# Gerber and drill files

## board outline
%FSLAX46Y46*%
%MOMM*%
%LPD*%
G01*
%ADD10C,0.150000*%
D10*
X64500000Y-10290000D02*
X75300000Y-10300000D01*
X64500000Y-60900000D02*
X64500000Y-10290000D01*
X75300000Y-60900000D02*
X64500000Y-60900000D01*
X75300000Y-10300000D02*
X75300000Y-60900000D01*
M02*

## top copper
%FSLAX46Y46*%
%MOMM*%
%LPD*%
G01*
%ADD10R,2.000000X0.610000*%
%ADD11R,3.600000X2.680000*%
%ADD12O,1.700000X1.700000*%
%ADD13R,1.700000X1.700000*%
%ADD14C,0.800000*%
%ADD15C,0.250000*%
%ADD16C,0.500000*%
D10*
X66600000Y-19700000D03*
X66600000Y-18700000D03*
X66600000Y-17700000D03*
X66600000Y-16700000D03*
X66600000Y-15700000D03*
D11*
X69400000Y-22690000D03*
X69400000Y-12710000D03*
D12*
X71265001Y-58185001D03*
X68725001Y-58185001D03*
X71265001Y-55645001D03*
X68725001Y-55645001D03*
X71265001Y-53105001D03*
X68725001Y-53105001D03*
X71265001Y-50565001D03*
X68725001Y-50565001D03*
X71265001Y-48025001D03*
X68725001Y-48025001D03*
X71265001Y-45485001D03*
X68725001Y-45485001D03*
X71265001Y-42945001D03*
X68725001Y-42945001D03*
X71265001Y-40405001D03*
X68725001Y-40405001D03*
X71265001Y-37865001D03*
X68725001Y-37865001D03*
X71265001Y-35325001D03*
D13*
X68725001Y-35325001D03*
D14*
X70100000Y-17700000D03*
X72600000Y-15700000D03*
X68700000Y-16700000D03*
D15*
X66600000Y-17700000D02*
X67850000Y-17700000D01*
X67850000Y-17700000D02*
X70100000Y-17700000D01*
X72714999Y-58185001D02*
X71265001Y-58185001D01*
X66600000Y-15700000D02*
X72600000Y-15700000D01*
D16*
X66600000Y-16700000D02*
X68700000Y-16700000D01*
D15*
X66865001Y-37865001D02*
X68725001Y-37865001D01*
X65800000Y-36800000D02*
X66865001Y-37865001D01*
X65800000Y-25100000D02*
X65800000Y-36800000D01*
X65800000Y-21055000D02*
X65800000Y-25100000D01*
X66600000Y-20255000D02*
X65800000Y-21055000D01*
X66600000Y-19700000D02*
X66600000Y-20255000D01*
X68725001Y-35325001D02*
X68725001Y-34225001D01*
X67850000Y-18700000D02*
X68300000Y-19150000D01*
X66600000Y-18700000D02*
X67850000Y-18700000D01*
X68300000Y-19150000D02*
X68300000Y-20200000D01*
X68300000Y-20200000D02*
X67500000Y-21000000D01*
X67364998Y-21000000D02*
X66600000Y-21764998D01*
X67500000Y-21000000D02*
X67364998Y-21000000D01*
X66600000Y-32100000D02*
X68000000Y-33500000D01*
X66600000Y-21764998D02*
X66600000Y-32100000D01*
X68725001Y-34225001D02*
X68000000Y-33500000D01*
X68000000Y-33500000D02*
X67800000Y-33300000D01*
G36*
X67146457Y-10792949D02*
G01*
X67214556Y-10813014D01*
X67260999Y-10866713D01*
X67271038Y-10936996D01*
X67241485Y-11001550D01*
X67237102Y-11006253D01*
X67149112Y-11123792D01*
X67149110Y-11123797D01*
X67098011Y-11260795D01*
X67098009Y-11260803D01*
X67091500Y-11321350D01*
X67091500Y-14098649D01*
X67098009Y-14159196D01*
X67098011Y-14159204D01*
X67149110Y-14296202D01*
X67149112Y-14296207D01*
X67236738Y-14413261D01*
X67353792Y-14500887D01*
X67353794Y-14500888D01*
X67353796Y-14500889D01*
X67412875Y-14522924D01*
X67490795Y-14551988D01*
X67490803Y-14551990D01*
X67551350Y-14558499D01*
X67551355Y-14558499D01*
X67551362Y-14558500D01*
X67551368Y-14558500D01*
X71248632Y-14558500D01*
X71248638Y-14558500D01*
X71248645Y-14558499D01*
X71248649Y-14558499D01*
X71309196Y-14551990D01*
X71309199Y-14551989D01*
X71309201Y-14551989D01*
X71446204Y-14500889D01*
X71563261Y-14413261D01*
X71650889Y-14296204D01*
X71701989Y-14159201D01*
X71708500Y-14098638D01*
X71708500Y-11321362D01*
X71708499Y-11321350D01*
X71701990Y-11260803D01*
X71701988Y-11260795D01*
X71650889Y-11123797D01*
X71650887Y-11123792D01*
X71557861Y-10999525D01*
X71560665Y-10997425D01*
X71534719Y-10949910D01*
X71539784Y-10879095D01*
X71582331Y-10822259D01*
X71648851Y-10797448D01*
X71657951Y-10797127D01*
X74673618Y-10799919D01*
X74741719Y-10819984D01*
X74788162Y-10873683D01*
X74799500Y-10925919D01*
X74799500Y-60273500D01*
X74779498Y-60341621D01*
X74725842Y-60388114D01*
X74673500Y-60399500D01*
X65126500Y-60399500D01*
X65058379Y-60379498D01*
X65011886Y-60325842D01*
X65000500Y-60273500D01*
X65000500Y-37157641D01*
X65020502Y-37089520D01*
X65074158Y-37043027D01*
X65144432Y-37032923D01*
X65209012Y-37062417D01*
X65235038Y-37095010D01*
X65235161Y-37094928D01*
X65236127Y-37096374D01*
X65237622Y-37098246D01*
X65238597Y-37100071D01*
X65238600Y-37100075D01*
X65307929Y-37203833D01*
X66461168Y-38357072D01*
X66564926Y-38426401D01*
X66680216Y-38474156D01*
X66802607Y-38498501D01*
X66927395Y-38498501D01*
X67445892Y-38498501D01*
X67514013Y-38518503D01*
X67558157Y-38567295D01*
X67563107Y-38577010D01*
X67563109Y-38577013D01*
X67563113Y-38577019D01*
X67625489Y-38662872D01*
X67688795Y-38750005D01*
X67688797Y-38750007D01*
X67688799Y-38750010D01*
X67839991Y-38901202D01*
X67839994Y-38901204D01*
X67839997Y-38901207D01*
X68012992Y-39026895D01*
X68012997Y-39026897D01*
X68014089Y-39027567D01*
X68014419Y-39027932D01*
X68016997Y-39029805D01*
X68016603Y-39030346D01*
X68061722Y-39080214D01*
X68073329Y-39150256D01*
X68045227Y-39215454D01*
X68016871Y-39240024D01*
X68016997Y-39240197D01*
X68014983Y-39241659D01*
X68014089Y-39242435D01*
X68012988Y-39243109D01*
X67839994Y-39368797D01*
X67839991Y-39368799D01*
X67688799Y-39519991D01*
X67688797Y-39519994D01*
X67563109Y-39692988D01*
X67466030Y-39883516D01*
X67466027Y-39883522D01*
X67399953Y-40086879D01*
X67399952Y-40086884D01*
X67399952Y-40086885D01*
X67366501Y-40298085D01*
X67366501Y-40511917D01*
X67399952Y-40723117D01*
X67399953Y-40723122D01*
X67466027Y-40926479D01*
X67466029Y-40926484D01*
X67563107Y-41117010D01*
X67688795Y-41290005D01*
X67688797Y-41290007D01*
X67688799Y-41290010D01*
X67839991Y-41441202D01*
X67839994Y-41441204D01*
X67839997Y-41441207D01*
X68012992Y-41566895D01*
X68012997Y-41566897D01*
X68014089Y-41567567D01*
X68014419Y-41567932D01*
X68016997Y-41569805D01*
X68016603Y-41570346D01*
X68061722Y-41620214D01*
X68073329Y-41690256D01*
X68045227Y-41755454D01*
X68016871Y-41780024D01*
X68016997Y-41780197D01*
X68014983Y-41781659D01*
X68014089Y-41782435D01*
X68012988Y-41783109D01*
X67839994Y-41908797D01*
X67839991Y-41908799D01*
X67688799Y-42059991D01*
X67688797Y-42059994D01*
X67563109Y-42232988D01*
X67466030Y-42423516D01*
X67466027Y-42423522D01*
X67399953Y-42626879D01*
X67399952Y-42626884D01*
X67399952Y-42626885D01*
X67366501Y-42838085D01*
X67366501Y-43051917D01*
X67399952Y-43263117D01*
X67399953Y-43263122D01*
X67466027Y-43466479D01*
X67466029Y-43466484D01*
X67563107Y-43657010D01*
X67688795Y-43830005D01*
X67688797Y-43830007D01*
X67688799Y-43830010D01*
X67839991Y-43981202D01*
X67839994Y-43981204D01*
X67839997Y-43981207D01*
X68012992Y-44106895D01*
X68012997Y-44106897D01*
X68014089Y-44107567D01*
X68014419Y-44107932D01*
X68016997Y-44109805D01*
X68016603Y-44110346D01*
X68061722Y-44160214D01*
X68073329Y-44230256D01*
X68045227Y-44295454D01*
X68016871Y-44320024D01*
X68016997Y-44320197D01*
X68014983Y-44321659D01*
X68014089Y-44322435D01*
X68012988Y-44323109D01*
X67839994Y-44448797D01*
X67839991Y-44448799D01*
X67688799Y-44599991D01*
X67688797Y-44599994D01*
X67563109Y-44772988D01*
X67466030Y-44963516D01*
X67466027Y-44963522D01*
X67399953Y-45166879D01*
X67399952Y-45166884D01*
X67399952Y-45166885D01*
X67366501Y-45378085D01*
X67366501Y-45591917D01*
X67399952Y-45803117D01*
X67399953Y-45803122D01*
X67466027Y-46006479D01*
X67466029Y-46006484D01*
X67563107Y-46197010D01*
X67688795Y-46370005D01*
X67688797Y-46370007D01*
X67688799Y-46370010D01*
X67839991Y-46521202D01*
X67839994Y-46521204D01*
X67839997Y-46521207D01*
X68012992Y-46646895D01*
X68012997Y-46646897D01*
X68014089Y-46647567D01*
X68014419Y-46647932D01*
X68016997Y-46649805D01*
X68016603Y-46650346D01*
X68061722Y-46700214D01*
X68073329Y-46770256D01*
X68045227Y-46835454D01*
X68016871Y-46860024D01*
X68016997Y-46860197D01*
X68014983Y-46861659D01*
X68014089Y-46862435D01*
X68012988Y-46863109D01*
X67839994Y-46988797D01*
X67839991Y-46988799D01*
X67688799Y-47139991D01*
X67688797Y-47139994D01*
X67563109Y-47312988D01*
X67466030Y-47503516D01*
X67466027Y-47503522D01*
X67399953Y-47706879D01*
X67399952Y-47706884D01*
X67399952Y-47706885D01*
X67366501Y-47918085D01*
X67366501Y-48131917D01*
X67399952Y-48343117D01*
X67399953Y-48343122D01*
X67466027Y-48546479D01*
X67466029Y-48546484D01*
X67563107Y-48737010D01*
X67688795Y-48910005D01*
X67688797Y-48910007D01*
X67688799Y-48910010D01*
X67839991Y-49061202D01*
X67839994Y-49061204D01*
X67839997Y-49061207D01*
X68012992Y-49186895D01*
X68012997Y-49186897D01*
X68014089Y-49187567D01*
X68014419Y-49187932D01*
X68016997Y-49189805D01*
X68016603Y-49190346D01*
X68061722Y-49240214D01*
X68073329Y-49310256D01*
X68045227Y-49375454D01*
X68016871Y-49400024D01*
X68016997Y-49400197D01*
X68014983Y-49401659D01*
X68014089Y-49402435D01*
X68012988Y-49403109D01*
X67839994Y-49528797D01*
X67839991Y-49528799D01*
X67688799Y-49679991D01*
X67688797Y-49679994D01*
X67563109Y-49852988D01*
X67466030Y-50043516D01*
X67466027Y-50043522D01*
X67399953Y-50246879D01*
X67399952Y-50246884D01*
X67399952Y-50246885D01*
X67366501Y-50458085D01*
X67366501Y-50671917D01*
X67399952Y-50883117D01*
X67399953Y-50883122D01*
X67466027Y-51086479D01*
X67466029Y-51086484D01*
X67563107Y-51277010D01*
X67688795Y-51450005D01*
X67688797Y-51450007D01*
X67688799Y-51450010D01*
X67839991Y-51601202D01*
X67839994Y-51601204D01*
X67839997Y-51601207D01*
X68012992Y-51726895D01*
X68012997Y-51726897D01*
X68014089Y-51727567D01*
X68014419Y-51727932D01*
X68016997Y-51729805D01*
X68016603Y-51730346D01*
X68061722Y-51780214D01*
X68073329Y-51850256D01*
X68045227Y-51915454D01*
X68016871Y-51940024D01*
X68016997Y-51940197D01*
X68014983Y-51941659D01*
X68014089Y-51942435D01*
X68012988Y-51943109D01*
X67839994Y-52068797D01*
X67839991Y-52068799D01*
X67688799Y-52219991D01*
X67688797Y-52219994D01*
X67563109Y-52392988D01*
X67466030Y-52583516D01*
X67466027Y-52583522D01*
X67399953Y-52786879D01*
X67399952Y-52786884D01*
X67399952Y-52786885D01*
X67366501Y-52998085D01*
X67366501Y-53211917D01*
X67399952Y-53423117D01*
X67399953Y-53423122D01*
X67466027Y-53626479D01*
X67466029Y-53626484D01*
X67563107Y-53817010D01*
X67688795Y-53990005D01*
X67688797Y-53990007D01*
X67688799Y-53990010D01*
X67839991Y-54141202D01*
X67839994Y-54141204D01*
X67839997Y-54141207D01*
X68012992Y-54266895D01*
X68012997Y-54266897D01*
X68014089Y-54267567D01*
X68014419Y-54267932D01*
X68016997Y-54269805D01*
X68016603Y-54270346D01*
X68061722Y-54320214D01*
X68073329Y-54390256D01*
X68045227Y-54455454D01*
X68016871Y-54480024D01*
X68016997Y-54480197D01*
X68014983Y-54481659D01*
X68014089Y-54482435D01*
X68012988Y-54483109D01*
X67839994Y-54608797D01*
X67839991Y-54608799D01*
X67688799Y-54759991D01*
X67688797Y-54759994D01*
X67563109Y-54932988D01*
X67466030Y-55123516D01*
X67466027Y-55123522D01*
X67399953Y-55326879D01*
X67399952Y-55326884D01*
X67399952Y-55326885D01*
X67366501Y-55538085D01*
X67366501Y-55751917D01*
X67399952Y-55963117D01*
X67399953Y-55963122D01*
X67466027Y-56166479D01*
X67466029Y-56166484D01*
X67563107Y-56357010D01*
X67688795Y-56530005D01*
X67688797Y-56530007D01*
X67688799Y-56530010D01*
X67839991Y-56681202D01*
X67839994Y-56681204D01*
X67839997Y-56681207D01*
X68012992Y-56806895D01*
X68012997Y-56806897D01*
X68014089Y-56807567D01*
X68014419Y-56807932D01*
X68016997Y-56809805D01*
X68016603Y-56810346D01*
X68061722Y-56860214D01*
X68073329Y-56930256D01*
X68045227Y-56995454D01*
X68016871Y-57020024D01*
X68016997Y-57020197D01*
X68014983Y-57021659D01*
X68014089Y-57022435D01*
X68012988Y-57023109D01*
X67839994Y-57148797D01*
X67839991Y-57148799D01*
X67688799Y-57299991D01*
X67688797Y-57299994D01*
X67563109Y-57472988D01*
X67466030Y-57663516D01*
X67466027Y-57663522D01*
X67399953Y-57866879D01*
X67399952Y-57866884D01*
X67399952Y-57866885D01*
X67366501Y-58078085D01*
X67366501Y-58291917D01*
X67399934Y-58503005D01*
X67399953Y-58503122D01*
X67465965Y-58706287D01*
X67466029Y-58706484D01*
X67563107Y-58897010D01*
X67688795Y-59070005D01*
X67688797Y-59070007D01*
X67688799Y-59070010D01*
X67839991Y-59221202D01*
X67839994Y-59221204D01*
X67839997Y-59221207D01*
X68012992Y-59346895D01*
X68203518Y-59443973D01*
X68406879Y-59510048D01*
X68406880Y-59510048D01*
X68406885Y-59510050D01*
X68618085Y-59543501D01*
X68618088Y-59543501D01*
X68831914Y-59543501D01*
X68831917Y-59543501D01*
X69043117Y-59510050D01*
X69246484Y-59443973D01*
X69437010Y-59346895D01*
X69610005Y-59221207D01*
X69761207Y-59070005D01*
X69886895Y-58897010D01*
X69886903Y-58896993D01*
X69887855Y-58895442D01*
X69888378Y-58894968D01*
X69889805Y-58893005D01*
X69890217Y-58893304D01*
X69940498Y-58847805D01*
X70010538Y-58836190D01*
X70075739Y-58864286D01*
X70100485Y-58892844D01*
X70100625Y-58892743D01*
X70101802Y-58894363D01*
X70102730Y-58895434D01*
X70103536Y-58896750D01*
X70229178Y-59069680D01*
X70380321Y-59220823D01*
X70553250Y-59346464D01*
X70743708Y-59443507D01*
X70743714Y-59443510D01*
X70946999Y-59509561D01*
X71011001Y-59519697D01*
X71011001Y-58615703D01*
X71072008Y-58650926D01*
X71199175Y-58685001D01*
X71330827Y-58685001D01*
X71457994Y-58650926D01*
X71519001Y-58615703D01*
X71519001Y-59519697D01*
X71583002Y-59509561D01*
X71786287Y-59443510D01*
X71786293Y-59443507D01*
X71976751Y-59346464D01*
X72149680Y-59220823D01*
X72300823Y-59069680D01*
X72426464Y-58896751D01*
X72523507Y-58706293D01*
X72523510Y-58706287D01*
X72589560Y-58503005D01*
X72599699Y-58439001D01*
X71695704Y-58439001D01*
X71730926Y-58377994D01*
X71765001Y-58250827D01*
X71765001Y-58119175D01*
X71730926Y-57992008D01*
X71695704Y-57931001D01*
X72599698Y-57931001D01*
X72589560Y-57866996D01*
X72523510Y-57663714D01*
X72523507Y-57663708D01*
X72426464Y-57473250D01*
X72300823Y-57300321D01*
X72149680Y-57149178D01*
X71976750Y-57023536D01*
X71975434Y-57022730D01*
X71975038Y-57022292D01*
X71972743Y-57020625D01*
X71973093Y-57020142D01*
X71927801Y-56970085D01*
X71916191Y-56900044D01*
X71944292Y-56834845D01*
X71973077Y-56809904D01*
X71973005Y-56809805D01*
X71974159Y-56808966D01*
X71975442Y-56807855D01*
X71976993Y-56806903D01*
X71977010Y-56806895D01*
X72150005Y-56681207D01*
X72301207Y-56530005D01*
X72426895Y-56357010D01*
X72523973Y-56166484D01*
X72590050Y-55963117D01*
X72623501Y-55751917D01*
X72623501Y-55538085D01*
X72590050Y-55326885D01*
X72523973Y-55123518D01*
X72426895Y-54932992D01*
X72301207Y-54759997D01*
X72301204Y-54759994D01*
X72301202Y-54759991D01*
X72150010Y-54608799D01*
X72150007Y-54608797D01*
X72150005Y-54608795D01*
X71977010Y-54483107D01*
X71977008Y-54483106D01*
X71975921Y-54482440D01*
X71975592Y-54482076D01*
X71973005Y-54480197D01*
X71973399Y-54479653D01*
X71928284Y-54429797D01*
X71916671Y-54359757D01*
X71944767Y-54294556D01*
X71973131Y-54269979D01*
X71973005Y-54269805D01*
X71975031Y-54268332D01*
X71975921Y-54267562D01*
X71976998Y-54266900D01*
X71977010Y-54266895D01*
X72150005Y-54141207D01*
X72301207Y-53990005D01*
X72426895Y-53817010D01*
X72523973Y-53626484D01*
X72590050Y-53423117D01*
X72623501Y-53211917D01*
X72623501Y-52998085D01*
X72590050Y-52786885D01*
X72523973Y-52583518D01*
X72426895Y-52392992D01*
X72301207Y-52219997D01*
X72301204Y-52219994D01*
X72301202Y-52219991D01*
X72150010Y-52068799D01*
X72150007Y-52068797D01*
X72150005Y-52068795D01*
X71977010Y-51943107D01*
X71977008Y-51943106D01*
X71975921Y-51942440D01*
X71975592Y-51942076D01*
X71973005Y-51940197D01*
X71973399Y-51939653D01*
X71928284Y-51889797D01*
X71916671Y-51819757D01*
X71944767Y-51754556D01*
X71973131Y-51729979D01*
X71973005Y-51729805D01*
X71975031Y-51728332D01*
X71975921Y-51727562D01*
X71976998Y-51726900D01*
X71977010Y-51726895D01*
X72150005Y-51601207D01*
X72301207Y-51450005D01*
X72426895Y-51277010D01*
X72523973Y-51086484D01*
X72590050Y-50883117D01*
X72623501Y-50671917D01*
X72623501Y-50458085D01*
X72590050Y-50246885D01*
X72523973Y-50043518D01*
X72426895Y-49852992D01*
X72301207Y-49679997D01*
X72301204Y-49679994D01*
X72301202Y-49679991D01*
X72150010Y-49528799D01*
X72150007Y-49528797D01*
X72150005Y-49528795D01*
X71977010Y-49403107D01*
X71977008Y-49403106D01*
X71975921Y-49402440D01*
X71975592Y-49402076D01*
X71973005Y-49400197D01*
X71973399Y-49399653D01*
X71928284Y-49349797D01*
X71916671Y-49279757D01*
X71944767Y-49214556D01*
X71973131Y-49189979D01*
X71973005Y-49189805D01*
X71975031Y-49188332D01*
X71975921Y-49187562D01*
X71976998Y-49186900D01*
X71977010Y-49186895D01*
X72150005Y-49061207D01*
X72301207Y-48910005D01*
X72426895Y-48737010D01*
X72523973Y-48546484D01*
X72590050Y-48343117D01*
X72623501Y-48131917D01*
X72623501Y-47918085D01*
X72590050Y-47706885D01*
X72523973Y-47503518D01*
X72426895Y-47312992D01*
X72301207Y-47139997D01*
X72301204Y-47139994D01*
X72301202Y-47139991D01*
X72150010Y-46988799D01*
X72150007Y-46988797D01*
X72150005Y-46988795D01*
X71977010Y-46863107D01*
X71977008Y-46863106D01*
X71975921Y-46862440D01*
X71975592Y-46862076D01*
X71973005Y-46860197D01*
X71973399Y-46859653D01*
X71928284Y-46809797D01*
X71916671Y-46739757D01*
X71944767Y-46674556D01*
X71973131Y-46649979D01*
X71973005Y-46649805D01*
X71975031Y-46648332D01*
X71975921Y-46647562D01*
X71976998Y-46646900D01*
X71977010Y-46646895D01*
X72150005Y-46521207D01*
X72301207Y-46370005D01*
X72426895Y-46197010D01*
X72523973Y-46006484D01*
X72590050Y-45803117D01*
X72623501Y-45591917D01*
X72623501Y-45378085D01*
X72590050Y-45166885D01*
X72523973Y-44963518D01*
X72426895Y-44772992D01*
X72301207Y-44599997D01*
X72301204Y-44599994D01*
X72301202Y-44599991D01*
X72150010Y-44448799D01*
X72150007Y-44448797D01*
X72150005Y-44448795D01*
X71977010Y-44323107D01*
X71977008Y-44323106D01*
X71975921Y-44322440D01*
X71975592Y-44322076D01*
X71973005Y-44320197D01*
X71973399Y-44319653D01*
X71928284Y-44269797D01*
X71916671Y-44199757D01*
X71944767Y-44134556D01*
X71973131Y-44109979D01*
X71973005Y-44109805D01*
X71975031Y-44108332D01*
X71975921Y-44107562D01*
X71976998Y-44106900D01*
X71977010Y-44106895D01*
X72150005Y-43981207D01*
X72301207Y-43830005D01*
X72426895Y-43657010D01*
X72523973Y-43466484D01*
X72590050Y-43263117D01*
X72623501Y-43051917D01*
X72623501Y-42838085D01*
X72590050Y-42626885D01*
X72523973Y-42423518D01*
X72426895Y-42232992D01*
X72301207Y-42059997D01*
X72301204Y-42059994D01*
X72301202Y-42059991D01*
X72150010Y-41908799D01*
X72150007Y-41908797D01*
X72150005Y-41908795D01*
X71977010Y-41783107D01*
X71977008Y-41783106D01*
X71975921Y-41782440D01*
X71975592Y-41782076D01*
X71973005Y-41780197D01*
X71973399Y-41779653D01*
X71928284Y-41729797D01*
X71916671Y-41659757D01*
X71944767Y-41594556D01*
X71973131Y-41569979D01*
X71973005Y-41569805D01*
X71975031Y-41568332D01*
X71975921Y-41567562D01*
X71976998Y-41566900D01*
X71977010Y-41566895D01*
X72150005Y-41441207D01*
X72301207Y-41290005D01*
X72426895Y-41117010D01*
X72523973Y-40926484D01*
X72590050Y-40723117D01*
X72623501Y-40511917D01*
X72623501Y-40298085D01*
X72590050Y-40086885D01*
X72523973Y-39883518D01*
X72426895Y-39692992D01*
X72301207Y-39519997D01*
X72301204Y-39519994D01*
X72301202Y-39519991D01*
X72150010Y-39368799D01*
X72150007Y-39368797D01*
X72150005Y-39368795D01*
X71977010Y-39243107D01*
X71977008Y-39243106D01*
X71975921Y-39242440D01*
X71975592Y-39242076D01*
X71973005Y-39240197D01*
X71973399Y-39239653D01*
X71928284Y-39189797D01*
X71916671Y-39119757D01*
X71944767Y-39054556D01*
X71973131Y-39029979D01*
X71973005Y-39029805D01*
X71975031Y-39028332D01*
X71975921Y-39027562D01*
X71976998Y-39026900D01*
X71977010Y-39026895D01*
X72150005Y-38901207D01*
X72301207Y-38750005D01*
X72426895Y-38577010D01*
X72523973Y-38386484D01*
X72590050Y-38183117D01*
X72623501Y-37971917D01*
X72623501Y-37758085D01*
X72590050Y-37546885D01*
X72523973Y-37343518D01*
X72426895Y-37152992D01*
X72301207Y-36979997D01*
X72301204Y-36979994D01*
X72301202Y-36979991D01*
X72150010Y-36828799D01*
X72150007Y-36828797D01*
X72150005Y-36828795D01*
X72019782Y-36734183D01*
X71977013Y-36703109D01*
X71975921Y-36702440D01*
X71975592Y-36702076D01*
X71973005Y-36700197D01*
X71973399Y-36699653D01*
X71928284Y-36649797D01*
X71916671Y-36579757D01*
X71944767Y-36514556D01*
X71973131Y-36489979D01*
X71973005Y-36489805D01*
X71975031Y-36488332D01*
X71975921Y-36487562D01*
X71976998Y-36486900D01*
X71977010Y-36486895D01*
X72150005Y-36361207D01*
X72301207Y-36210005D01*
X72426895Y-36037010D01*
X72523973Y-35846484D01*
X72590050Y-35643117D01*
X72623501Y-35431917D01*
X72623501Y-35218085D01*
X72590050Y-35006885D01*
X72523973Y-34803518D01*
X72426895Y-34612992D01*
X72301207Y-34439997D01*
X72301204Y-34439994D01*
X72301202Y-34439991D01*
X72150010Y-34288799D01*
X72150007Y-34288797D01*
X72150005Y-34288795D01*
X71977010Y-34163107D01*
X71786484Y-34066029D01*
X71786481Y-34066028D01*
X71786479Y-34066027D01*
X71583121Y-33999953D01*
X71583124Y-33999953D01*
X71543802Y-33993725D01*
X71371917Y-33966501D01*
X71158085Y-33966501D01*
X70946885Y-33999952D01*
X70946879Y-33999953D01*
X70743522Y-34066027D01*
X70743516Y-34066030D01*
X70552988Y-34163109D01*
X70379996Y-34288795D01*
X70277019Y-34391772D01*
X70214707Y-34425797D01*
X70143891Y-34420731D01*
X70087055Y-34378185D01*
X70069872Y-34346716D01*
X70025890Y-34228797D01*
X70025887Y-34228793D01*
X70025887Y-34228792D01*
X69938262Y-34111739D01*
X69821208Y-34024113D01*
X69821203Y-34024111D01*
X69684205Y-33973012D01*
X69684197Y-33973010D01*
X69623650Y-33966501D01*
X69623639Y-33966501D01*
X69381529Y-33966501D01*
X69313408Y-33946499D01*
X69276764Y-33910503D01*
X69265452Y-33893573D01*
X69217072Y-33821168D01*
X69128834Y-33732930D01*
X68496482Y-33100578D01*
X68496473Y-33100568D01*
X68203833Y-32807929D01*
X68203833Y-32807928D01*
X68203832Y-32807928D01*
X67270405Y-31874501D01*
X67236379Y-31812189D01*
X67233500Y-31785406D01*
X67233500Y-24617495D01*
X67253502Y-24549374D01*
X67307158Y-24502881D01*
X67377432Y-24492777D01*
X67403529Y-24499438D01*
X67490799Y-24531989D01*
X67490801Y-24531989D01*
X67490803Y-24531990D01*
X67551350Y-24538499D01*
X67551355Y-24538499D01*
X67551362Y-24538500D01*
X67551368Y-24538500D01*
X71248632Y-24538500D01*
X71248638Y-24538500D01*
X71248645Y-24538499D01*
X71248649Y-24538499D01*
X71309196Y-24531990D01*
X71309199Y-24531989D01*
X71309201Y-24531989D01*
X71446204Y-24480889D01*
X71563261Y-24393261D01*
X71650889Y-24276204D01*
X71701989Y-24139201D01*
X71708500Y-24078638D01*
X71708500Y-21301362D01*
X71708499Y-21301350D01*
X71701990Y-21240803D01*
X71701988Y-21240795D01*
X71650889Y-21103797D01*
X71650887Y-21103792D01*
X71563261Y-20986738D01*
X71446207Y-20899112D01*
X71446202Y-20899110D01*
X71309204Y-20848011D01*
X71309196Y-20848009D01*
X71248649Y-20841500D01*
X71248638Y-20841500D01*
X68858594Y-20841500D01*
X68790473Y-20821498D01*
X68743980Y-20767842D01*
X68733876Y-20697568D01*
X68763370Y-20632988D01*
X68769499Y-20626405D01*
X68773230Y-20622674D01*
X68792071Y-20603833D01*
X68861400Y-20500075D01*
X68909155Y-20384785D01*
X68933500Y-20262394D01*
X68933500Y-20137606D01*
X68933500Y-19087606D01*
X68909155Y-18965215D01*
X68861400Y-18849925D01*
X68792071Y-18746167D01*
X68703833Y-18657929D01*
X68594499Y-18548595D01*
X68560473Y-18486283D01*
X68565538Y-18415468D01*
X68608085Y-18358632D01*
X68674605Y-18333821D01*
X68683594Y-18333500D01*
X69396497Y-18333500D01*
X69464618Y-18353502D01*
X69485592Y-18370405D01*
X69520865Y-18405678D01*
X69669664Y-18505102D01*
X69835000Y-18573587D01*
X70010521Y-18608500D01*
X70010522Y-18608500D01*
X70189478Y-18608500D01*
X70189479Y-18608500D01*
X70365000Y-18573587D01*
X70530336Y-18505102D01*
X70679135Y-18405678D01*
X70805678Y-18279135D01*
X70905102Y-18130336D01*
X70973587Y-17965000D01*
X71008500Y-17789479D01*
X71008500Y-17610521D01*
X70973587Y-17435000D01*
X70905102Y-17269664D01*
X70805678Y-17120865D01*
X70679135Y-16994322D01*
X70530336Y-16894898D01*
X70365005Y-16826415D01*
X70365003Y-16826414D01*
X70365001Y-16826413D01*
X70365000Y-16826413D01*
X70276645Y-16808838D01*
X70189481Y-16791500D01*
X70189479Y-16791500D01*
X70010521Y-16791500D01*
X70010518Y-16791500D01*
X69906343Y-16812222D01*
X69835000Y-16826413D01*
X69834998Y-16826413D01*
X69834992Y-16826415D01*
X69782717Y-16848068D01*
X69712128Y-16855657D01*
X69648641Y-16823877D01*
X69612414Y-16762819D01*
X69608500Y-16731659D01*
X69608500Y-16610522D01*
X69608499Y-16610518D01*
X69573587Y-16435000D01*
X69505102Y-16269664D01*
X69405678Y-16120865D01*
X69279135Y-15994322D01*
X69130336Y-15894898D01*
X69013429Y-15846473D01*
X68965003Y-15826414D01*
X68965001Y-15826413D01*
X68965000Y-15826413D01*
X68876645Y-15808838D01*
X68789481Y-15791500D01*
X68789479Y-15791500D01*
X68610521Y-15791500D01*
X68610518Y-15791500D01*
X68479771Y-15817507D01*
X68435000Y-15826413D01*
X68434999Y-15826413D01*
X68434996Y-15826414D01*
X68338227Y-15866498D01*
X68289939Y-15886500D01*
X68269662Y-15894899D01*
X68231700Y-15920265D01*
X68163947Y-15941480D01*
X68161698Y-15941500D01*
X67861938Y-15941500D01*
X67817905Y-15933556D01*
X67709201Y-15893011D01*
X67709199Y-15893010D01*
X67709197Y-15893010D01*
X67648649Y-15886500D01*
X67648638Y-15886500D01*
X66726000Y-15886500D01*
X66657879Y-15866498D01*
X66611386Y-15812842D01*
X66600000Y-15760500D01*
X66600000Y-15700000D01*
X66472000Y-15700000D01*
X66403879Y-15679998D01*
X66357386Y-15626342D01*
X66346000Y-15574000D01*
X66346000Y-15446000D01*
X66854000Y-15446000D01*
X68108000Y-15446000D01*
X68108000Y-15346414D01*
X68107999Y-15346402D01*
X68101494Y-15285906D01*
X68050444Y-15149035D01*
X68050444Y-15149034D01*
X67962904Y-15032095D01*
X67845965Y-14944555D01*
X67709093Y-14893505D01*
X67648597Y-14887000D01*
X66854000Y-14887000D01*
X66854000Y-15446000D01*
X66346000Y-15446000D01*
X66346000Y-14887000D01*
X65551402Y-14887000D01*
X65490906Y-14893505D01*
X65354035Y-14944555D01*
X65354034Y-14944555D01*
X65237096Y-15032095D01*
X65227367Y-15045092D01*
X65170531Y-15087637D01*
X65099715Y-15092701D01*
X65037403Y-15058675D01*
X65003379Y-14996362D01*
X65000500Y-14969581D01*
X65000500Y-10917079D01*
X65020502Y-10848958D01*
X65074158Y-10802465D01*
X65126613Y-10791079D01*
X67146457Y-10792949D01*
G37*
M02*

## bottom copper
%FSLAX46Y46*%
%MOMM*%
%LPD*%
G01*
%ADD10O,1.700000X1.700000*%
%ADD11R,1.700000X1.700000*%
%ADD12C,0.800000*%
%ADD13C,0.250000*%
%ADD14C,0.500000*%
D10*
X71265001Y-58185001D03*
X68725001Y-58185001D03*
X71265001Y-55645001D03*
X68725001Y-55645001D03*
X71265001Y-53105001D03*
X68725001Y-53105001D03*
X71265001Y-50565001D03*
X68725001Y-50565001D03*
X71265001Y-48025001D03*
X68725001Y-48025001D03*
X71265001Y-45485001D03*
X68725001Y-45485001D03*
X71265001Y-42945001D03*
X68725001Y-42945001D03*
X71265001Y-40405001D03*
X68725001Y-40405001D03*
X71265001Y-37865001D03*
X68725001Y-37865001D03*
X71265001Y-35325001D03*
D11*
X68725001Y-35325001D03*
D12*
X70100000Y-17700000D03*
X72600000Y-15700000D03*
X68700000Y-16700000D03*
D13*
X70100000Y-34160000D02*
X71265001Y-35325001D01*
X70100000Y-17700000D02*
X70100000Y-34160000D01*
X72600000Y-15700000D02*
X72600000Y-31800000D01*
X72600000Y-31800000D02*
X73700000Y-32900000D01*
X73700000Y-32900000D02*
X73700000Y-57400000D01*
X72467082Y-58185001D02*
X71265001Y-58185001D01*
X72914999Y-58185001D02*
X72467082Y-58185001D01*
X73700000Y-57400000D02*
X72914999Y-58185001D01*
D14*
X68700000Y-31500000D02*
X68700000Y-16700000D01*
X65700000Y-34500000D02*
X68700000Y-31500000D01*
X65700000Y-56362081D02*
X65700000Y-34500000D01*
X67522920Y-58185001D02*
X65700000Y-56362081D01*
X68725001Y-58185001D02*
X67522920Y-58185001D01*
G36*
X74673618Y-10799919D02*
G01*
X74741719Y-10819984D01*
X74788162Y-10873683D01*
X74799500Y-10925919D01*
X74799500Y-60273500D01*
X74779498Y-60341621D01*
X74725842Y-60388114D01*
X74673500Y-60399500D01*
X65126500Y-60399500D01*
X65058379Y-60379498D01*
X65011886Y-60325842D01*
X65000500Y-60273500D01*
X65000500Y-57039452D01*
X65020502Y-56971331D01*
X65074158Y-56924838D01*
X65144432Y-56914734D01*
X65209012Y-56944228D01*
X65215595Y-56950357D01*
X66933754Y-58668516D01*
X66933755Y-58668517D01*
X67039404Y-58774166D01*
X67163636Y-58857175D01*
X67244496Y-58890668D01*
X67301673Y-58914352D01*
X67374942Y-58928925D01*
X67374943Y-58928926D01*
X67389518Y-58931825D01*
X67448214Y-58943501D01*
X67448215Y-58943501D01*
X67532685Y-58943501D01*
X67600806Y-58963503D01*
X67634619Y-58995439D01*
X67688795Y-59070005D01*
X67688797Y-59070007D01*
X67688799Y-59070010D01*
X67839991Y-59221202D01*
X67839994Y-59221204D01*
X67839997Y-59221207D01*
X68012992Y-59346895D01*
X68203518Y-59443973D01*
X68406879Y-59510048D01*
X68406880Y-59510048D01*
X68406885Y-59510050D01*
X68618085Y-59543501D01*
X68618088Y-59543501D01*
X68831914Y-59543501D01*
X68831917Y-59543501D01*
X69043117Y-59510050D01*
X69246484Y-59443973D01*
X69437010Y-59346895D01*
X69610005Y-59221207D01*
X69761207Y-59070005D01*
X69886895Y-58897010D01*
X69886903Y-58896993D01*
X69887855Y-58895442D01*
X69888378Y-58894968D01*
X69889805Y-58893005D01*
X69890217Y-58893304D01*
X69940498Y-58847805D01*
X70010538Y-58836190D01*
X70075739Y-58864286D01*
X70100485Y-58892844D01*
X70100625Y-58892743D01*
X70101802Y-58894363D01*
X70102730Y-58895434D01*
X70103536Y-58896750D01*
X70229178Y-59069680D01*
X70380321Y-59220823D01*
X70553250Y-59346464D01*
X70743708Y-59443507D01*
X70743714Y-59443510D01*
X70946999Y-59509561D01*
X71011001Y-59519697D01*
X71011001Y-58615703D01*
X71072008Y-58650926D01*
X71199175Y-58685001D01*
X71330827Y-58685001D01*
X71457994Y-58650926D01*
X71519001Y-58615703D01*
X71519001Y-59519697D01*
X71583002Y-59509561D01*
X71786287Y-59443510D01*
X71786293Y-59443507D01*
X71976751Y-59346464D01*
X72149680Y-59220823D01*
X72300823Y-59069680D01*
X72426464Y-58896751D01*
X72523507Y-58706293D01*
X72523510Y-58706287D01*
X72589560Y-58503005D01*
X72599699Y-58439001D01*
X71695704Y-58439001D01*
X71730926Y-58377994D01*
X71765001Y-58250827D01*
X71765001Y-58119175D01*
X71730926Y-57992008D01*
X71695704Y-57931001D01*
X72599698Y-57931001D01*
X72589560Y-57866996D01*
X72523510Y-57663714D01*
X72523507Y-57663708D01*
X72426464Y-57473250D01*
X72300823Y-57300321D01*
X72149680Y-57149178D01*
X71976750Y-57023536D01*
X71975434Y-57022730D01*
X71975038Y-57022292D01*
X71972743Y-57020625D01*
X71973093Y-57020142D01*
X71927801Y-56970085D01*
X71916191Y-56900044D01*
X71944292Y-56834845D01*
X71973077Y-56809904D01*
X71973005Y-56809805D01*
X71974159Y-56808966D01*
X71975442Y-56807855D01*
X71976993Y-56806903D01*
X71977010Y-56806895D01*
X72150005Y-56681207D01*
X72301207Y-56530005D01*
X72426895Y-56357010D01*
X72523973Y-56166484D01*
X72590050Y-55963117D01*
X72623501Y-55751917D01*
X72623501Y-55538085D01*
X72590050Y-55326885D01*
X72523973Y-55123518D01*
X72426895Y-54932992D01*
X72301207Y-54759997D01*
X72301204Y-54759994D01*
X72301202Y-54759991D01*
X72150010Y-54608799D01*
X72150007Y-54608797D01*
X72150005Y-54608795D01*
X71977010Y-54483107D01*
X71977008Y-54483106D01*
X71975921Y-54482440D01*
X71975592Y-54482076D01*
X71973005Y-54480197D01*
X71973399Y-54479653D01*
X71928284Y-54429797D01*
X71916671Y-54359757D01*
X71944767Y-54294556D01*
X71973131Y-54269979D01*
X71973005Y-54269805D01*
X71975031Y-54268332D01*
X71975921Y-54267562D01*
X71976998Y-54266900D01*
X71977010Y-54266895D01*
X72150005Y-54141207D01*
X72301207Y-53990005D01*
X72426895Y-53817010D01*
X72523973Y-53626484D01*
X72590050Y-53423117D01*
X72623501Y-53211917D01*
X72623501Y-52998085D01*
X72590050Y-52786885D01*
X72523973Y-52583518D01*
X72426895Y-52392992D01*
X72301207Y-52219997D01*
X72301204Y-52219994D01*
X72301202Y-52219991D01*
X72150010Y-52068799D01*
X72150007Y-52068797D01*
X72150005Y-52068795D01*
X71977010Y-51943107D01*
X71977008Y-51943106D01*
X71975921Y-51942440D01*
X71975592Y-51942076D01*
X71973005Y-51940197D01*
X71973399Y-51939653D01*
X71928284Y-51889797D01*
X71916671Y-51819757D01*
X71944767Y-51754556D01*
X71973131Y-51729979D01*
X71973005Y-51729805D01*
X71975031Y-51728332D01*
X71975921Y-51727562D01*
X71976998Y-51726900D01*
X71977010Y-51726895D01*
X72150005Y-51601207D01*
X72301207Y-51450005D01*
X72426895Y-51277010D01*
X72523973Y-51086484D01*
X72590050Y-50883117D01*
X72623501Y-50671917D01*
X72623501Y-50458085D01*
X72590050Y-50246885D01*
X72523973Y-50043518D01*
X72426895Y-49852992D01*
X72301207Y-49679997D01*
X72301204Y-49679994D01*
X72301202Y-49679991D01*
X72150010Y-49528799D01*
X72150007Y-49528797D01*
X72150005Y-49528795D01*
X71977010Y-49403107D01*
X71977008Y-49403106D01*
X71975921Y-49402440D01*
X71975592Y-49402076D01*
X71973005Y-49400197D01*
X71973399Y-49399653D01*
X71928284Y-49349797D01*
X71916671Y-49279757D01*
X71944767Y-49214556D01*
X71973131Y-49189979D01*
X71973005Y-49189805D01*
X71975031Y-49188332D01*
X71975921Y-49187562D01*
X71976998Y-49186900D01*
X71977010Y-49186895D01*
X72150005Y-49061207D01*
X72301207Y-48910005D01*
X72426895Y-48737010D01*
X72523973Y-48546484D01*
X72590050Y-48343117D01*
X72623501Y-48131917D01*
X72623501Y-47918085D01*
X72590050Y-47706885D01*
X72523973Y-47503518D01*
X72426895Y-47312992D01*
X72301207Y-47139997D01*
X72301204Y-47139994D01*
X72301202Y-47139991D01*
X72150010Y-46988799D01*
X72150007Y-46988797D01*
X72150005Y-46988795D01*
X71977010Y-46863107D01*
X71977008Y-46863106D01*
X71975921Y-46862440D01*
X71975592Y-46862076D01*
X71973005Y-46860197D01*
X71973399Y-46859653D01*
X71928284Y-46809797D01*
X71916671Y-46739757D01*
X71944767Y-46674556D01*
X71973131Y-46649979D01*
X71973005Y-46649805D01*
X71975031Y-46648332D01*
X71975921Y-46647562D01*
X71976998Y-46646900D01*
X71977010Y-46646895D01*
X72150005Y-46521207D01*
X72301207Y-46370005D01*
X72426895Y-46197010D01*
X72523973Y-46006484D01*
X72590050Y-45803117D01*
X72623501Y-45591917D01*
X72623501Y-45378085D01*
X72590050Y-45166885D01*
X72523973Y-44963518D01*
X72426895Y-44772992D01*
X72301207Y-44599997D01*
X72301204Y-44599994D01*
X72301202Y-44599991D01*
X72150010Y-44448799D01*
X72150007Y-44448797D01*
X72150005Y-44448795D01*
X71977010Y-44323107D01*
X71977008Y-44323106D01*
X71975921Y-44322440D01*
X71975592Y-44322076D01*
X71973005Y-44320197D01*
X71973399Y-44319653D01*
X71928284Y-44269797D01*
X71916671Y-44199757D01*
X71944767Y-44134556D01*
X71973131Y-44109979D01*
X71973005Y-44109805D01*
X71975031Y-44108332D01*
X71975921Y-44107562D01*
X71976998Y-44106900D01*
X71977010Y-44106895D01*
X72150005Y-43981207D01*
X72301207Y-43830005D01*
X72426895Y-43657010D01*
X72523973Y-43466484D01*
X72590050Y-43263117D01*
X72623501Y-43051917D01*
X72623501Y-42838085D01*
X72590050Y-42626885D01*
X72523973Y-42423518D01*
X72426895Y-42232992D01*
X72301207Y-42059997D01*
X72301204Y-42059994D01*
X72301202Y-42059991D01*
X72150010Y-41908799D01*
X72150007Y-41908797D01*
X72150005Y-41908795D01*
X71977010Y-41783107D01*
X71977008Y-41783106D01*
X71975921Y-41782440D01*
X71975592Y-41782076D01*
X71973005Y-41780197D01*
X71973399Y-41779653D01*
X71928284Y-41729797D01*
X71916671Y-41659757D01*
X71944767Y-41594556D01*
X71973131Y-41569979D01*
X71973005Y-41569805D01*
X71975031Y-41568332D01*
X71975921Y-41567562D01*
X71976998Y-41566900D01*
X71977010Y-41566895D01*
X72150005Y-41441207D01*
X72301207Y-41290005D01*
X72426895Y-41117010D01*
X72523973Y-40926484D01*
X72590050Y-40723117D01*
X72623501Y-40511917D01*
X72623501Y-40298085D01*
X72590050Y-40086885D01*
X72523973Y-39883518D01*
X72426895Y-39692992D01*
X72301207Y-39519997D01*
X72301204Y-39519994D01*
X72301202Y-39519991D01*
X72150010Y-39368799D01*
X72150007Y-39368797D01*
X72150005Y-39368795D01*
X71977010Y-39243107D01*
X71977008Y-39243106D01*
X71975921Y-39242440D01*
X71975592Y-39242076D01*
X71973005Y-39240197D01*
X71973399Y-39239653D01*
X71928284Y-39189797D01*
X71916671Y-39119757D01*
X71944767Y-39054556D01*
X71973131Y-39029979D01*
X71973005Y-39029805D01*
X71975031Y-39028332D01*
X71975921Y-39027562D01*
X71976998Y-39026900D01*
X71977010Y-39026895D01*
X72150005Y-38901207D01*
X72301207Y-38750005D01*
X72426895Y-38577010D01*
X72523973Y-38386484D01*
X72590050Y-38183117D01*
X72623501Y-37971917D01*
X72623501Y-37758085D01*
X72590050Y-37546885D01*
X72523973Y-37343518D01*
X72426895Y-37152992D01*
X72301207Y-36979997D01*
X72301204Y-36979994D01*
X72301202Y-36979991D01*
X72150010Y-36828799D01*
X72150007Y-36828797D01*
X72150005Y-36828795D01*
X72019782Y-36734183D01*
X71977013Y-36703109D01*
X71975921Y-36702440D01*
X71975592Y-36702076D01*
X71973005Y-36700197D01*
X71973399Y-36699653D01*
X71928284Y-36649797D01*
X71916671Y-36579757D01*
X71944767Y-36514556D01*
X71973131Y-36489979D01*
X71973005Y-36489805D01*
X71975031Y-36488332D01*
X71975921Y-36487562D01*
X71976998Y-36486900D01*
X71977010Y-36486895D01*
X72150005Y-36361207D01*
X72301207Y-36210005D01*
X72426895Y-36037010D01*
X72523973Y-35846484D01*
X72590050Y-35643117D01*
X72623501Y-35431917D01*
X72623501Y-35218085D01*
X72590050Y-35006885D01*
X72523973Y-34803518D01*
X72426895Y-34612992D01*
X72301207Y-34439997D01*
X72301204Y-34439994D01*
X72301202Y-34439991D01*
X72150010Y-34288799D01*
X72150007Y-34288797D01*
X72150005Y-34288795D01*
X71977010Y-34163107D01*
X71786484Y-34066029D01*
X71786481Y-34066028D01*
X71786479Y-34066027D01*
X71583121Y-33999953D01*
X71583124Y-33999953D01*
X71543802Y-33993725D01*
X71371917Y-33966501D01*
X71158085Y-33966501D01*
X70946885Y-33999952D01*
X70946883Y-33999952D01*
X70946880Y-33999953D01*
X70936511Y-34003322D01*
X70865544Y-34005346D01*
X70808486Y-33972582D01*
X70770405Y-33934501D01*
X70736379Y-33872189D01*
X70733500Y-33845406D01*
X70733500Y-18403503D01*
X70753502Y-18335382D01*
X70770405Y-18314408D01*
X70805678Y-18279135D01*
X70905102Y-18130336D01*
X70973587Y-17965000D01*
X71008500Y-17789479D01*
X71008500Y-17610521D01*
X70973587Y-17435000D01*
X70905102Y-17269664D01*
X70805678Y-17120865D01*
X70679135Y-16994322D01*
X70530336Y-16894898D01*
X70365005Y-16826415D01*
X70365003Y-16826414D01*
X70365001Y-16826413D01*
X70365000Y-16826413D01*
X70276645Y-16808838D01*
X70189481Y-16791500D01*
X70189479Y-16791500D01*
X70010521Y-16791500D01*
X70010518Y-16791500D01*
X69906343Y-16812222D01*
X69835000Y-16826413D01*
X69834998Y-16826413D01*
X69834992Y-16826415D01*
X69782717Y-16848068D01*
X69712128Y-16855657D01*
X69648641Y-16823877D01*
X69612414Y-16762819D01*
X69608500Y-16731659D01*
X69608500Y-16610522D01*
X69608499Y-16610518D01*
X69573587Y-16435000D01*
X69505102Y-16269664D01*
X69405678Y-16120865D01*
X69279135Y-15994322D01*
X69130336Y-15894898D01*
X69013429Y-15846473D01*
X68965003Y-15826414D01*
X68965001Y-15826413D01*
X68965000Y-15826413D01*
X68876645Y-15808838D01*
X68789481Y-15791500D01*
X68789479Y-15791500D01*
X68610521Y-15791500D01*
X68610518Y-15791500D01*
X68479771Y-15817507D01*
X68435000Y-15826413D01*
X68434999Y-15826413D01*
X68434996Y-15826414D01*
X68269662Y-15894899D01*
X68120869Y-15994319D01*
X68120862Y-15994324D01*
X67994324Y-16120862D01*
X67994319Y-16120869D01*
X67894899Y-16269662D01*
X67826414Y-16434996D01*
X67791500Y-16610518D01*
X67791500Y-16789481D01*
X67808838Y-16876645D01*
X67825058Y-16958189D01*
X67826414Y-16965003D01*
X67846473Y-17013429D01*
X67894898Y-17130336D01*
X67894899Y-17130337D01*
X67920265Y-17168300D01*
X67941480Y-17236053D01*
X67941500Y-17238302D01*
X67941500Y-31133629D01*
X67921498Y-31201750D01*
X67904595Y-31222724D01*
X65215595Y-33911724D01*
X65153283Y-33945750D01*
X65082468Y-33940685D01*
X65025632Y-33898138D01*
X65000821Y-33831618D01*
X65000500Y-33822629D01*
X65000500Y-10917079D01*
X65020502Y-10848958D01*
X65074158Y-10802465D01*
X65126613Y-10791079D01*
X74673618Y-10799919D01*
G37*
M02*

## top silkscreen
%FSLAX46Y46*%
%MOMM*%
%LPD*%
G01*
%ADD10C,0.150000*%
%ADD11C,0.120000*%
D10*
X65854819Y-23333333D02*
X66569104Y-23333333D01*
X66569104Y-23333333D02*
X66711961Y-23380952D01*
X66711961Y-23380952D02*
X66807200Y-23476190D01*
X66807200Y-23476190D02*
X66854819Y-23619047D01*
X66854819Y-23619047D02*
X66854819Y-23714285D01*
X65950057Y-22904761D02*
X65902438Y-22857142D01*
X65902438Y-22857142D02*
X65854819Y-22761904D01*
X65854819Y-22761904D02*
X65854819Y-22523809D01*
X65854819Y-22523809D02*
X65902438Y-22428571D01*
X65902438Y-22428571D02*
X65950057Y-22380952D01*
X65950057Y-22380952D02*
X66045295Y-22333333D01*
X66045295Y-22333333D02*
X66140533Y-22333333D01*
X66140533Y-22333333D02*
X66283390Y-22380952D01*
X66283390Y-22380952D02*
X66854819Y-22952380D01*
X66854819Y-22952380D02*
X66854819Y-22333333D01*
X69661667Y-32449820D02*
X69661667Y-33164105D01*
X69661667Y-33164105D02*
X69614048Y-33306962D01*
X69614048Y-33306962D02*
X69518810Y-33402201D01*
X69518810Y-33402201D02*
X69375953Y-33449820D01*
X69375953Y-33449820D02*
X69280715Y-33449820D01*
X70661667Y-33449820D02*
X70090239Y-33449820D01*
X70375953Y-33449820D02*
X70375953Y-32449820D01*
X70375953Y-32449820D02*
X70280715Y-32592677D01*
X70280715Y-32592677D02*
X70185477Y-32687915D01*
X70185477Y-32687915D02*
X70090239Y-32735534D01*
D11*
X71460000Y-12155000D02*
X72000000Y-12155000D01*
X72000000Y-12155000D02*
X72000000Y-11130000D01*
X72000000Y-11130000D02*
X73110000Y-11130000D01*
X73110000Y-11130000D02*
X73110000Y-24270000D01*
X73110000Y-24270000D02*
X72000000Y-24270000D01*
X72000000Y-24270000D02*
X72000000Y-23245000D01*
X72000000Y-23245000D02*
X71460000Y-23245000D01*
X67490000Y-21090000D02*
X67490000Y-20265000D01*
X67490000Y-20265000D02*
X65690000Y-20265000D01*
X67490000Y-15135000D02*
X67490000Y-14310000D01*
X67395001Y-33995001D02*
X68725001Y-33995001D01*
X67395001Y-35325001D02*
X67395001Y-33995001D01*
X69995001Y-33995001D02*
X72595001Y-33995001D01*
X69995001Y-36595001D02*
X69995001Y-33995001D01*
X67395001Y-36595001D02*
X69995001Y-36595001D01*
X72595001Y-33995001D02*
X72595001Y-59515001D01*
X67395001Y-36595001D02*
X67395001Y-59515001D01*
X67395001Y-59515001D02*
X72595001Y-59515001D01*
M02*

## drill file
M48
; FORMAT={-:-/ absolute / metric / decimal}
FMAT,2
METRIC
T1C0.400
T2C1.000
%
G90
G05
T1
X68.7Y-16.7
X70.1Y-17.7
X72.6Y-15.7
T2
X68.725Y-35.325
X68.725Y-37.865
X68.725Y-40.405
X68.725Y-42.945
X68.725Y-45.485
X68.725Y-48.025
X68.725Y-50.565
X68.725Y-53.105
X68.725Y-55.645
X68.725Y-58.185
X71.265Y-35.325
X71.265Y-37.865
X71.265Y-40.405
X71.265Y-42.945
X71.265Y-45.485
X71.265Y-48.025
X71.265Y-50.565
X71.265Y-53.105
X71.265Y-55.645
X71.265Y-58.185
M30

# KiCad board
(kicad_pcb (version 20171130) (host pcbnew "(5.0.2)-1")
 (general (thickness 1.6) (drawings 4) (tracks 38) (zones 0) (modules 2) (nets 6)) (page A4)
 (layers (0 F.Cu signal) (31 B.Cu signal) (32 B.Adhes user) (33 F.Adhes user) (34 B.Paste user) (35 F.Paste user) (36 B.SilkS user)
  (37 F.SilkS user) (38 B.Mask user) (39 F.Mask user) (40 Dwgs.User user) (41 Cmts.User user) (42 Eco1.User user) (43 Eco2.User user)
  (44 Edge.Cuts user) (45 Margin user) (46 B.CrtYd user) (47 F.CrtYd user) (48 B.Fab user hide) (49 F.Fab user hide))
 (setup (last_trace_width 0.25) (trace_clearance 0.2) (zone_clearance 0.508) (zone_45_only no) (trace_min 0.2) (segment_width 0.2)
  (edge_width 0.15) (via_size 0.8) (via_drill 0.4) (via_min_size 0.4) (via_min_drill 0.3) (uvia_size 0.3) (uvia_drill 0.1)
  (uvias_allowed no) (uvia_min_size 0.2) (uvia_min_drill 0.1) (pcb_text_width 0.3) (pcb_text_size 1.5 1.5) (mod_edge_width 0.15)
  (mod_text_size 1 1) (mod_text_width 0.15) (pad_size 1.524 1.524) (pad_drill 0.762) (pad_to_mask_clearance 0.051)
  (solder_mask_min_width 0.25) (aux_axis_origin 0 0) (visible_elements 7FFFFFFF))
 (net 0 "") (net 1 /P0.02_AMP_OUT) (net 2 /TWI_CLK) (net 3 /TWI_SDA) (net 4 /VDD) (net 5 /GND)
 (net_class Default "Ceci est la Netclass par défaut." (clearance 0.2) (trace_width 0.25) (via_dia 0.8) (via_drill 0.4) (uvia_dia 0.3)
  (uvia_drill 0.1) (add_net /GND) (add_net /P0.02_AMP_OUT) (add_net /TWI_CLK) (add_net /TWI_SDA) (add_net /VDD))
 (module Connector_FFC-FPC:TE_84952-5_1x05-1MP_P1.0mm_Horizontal (layer F.Cu) (at 68.4 17.7 90)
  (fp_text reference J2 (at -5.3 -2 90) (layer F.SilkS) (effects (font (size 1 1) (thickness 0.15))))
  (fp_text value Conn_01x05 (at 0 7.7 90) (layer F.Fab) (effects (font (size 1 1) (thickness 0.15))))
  (fp_line (start 5.545 3.06) (end 5.545 3.6) (layer F.SilkS) (width 0.12))
  (fp_line (start 5.545 3.6) (end 6.57 3.6) (layer F.SilkS) (width 0.12))
  (fp_line (start 6.57 3.6) (end 6.57 4.71) (layer F.SilkS) (width 0.12))
  (fp_line (start 6.57 4.71) (end -6.57 4.71) (layer F.SilkS) (width 0.12))
  (fp_line (start -6.57 4.71) (end -6.57 3.6) (layer F.SilkS) (width 0.12))
  (fp_line (start -6.57 3.6) (end -5.545 3.6) (layer F.SilkS) (width 0.12))
  (fp_line (start -5.545 3.6) (end -5.545 3.06) (layer F.SilkS) (width 0.12))
  (fp_line (start -3.39 -0.91) (end -2.565 -0.91) (layer F.SilkS) (width 0.12))
  (fp_line (start -2.565 -0.91) (end -2.565 -2.71) (layer F.SilkS) (width 0.12))
  (fp_line (start 2.565 -0.91) (end 3.39 -0.91) (layer F.SilkS) (width 0.12))
  (pad 1 smd rect (at -2 -1.8 90) (size 0.61 2) (layers F.Cu F.Paste F.Mask) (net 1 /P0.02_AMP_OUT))
  (pad 2 smd rect (at -1 -1.8 90) (size 0.61 2) (layers F.Cu F.Paste F.Mask) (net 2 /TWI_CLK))
  (pad 3 smd rect (at 0 -1.8 90) (size 0.61 2) (layers F.Cu F.Paste F.Mask) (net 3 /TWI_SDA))
  (pad 4 smd rect (at 1 -1.8 90) (size 0.61 2) (layers F.Cu F.Paste F.Mask) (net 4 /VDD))
  (pad 5 smd rect (at 2 -1.8 90) (size 0.61 2) (layers F.Cu F.Paste F.Mask) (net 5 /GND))
  (pad MP smd rect (at -4.99 1 90) (size 2.68 3.6) (layers F.Cu F.Paste F.Mask))
  (pad MP smd rect (at 4.99 1 90) (size 2.68 3.6) (layers F.Cu F.Paste F.Mask)))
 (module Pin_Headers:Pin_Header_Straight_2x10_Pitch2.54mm (layer F.Cu) (at 68.725001 35.325001)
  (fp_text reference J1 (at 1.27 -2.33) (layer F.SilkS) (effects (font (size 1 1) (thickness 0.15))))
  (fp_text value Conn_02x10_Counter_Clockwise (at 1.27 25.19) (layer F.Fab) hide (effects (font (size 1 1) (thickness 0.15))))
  (fp_line (start -1.33 -1.33) (end 0 -1.33) (layer F.SilkS) (width 0.12))
  (fp_line (start -1.33 0) (end -1.33 -1.33) (layer F.SilkS) (width 0.12))
  (fp_line (start 1.27 -1.33) (end 3.87 -1.33) (layer F.SilkS) (width 0.12))
  (fp_line (start 1.27 1.27) (end 1.27 -1.33) (layer F.SilkS) (width 0.12))
  (fp_line (start -1.33 1.27) (end 1.27 1.27) (layer F.SilkS) (width 0.12))
  (fp_line (start 3.87 -1.33) (end 3.87 24.19) (layer F.SilkS) (width 0.12))
  (fp_line (start -1.33 1.27) (end -1.33 24.19) (layer F.SilkS) (width 0.12))
  (fp_line (start -1.33 24.19) (end 3.87 24.19) (layer F.SilkS) (width 0.12))
  (pad 20 thru_hole oval (at 2.54 22.86) (size 1.7 1.7) (drill 1) (layers *.Cu *.Mask) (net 5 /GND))
  (pad 19 thru_hole oval (at 0 22.86) (size 1.7 1.7) (drill 1) (layers *.Cu *.Mask) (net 4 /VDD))
  (pad 18 thru_hole oval (at 2.54 20.32) (size 1.7 1.7) (drill 1) (layers *.Cu *.Mask))
  (pad 17 thru_hole oval (at 0 20.32) (size 1.7 1.7) (drill 1) (layers *.Cu *.Mask))
  (pad 16 thru_hole oval (at 2.54 17.78) (size 1.7 1.7) (drill 1) (layers *.Cu *.Mask))
  (pad 15 thru_hole oval (at 0 17.78) (size 1.7 1.7) (drill 1) (layers *.Cu *.Mask))
  (pad 14 thru_hole oval (at 2.54 15.24) (size 1.7 1.7) (drill 1) (layers *.Cu *.Mask))
  (pad 13 thru_hole oval (at 0 15.24) (size 1.7 1.7) (drill 1) (layers *.Cu *.Mask))
  (pad 12 thru_hole oval (at 2.54 12.7) (size 1.7 1.7) (drill 1) (layers *.Cu *.Mask))
  (pad 11 thru_hole oval (at 0 12.7) (size 1.7 1.7) (drill 1) (layers *.Cu *.Mask))
  (pad 10 thru_hole oval (at 2.54 10.16) (size 1.7 1.7) (drill 1) (layers *.Cu *.Mask))
  (pad 9 thru_hole oval (at 0 10.16) (size 1.7 1.7) (drill 1) (layers *.Cu *.Mask))
  (pad 8 thru_hole oval (at 2.54 7.62) (size 1.7 1.7) (drill 1) (layers *.Cu *.Mask))
  (pad 7 thru_hole oval (at 0 7.62) (size 1.7 1.7) (drill 1) (layers *.Cu *.Mask))
  (pad 6 thru_hole oval (at 2.54 5.08) (size 1.7 1.7) (drill 1) (layers *.Cu *.Mask))
  (pad 5 thru_hole oval (at 0 5.08) (size 1.7 1.7) (drill 1) (layers *.Cu *.Mask))
  (pad 4 thru_hole oval (at 2.54 2.54) (size 1.7 1.7) (drill 1) (layers *.Cu *.Mask))
  (pad 3 thru_hole oval (at 0 2.54) (size 1.7 1.7) (drill 1) (layers *.Cu *.Mask) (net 1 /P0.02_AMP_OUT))
  (pad 2 thru_hole oval (at 2.54 0) (size 1.7 1.7) (drill 1) (layers *.Cu *.Mask) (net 3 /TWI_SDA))
  (pad 1 thru_hole rect (at 0 0) (size 1.7 1.7) (drill 1) (layers *.Cu *.Mask) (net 2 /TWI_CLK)))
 (gr_line (start 64.5 10.29) (end 75.3 10.3) (layer Edge.Cuts) (width 0.15))
 (gr_line (start 64.5 60.9) (end 64.5 10.29) (layer Edge.Cuts) (width 0.15))
 (gr_line (start 75.3 60.9) (end 64.5 60.9) (layer Edge.Cuts) (width 0.15))
 (gr_line (start 75.3 10.3) (end 75.3 60.9) (layer Edge.Cuts) (width 0.15))
 (segment (start 66.6 17.7) (end 67.85 17.7) (width 0.25) (layer F.Cu) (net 3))
 (segment (start 67.85 17.7) (end 70.1 17.7) (width 0.25) (layer F.Cu) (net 3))
 (via (at 70.1 17.7) (size 0.8) (drill 0.4) (layers F.Cu B.Cu) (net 3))
 (segment (start 70.1 34.16) (end 71.265001 35.325001) (width 0.25) (layer B.Cu) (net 3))
 (segment (start 70.1 17.7) (end 70.1 34.16) (width 0.25) (layer B.Cu) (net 3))
 (segment (start 72.714999 58.185001) (end 71.265001 58.185001) (width 0.25) (layer F.Cu) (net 5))
 (via (at 72.6 15.7) (size 0.8) (drill 0.4) (layers F.Cu B.Cu) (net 5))
 (segment (start 66.6 15.7) (end 72.6 15.7) (width 0.25) (layer F.Cu) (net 5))
 (segment (start 72.6 15.7) (end 72.6 31.8) (width 0.25) (layer B.Cu) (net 5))
 (segment (start 72.6 31.8) (end 73.7 32.9) (width 0.25) (layer B.Cu) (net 5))
 (segment (start 73.7 32.9) (end 73.7 57.4) (width 0.25) (layer B.Cu) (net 5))
 (segment (start 72.467082 58.185001) (end 71.265001 58.185001) (width 0.25) (layer B.Cu) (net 5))
 (segment (start 72.914999 58.185001) (end 72.467082 58.185001) (width 0.25) (layer B.Cu) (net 5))
 (segment (start 73.7 57.4) (end 72.914999 58.185001) (width 0.25) (layer B.Cu) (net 5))
 (via (at 68.7 16.7) (size 0.8) (drill 0.4) (layers F.Cu B.Cu) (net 4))
 (segment (start 66.6 16.7) (end 68.7 16.7) (width 0.5) (layer F.Cu) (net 4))
 (segment (start 68.7 31.5) (end 68.7 16.7) (width 0.5) (layer B.Cu) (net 4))
 (segment (start 65.7 34.5) (end 68.7 31.5) (width 0.5) (layer B.Cu) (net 4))
 (segment (start 65.7 56.362081) (end 65.7 34.5) (width 0.5) (layer B.Cu) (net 4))
 (segment (start 67.52292 58.185001) (end 65.7 56.362081) (width 0.5) (layer B.Cu) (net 4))
 (segment (start 68.725001 58.185001) (end 67.52292 58.185001) (width 0.5) (layer B.Cu) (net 4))
 (segment (start 66.865001 37.865001) (end 68.725001 37.865001) (width 0.25) (layer F.Cu) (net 1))
 (segment (start 65.8 36.8) (end 66.865001 37.865001) (width 0.25) (layer F.Cu) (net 1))
 (segment (start 65.8 25.1) (end 65.8 36.8) (width 0.25) (layer F.Cu) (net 1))
 (segment (start 65.8 21.055) (end 65.8 25.1) (width 0.25) (layer F.Cu) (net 1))
 (segment (start 66.6 20.255) (end 65.8 21.055) (width 0.25) (layer F.Cu) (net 1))
 (segment (start 66.6 19.7) (end 66.6 20.255) (width 0.25) (layer F.Cu) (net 1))
 (segment (start 68.725001 35.325001) (end 68.725001 34.225001) (width 0.25) (layer F.Cu) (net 2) (status 10))
 (segment (start 67.85 18.7) (end 68.3 19.15) (width 0.25) (layer F.Cu) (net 2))
 (segment (start 66.6 18.7) (end 67.85 18.7) (width 0.25) (layer F.Cu) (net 2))
 (segment (start 68.3 19.15) (end 68.3 20.2) (width 0.25) (layer F.Cu) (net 2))
 (segment (start 68.3 20.2) (end 67.5 21) (width 0.25) (layer F.Cu) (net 2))
 (segment (start 67.364998 21) (end 66.6 21.764998) (width 0.25) (layer F.Cu) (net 2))
 (segment (start 67.5 21) (end 67.364998 21) (width 0.25) (layer F.Cu) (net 2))
 (segment (start 66.6 32.1) (end 68 33.5) (width 0.25) (layer F.Cu) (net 2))
 (segment (start 66.6 21.764998) (end 66.6 32.1) (width 0.25) (layer F.Cu) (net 2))
 (segment (start 68.725001 34.225001) (end 68 33.5) (width 0.25) (layer F.Cu) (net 2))
 (segment (start 68 33.5) (end 67.8 33.3) (width 0.25) (layer F.Cu) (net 2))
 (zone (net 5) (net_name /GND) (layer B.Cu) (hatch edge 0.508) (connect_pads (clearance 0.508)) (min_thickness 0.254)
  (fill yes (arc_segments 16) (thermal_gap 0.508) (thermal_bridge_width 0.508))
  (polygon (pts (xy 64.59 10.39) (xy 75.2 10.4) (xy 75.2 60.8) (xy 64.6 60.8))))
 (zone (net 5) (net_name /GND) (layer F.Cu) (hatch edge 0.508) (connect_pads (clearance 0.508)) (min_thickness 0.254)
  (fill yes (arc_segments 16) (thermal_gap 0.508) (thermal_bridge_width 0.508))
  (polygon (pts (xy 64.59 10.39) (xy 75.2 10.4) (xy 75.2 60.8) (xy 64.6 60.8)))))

